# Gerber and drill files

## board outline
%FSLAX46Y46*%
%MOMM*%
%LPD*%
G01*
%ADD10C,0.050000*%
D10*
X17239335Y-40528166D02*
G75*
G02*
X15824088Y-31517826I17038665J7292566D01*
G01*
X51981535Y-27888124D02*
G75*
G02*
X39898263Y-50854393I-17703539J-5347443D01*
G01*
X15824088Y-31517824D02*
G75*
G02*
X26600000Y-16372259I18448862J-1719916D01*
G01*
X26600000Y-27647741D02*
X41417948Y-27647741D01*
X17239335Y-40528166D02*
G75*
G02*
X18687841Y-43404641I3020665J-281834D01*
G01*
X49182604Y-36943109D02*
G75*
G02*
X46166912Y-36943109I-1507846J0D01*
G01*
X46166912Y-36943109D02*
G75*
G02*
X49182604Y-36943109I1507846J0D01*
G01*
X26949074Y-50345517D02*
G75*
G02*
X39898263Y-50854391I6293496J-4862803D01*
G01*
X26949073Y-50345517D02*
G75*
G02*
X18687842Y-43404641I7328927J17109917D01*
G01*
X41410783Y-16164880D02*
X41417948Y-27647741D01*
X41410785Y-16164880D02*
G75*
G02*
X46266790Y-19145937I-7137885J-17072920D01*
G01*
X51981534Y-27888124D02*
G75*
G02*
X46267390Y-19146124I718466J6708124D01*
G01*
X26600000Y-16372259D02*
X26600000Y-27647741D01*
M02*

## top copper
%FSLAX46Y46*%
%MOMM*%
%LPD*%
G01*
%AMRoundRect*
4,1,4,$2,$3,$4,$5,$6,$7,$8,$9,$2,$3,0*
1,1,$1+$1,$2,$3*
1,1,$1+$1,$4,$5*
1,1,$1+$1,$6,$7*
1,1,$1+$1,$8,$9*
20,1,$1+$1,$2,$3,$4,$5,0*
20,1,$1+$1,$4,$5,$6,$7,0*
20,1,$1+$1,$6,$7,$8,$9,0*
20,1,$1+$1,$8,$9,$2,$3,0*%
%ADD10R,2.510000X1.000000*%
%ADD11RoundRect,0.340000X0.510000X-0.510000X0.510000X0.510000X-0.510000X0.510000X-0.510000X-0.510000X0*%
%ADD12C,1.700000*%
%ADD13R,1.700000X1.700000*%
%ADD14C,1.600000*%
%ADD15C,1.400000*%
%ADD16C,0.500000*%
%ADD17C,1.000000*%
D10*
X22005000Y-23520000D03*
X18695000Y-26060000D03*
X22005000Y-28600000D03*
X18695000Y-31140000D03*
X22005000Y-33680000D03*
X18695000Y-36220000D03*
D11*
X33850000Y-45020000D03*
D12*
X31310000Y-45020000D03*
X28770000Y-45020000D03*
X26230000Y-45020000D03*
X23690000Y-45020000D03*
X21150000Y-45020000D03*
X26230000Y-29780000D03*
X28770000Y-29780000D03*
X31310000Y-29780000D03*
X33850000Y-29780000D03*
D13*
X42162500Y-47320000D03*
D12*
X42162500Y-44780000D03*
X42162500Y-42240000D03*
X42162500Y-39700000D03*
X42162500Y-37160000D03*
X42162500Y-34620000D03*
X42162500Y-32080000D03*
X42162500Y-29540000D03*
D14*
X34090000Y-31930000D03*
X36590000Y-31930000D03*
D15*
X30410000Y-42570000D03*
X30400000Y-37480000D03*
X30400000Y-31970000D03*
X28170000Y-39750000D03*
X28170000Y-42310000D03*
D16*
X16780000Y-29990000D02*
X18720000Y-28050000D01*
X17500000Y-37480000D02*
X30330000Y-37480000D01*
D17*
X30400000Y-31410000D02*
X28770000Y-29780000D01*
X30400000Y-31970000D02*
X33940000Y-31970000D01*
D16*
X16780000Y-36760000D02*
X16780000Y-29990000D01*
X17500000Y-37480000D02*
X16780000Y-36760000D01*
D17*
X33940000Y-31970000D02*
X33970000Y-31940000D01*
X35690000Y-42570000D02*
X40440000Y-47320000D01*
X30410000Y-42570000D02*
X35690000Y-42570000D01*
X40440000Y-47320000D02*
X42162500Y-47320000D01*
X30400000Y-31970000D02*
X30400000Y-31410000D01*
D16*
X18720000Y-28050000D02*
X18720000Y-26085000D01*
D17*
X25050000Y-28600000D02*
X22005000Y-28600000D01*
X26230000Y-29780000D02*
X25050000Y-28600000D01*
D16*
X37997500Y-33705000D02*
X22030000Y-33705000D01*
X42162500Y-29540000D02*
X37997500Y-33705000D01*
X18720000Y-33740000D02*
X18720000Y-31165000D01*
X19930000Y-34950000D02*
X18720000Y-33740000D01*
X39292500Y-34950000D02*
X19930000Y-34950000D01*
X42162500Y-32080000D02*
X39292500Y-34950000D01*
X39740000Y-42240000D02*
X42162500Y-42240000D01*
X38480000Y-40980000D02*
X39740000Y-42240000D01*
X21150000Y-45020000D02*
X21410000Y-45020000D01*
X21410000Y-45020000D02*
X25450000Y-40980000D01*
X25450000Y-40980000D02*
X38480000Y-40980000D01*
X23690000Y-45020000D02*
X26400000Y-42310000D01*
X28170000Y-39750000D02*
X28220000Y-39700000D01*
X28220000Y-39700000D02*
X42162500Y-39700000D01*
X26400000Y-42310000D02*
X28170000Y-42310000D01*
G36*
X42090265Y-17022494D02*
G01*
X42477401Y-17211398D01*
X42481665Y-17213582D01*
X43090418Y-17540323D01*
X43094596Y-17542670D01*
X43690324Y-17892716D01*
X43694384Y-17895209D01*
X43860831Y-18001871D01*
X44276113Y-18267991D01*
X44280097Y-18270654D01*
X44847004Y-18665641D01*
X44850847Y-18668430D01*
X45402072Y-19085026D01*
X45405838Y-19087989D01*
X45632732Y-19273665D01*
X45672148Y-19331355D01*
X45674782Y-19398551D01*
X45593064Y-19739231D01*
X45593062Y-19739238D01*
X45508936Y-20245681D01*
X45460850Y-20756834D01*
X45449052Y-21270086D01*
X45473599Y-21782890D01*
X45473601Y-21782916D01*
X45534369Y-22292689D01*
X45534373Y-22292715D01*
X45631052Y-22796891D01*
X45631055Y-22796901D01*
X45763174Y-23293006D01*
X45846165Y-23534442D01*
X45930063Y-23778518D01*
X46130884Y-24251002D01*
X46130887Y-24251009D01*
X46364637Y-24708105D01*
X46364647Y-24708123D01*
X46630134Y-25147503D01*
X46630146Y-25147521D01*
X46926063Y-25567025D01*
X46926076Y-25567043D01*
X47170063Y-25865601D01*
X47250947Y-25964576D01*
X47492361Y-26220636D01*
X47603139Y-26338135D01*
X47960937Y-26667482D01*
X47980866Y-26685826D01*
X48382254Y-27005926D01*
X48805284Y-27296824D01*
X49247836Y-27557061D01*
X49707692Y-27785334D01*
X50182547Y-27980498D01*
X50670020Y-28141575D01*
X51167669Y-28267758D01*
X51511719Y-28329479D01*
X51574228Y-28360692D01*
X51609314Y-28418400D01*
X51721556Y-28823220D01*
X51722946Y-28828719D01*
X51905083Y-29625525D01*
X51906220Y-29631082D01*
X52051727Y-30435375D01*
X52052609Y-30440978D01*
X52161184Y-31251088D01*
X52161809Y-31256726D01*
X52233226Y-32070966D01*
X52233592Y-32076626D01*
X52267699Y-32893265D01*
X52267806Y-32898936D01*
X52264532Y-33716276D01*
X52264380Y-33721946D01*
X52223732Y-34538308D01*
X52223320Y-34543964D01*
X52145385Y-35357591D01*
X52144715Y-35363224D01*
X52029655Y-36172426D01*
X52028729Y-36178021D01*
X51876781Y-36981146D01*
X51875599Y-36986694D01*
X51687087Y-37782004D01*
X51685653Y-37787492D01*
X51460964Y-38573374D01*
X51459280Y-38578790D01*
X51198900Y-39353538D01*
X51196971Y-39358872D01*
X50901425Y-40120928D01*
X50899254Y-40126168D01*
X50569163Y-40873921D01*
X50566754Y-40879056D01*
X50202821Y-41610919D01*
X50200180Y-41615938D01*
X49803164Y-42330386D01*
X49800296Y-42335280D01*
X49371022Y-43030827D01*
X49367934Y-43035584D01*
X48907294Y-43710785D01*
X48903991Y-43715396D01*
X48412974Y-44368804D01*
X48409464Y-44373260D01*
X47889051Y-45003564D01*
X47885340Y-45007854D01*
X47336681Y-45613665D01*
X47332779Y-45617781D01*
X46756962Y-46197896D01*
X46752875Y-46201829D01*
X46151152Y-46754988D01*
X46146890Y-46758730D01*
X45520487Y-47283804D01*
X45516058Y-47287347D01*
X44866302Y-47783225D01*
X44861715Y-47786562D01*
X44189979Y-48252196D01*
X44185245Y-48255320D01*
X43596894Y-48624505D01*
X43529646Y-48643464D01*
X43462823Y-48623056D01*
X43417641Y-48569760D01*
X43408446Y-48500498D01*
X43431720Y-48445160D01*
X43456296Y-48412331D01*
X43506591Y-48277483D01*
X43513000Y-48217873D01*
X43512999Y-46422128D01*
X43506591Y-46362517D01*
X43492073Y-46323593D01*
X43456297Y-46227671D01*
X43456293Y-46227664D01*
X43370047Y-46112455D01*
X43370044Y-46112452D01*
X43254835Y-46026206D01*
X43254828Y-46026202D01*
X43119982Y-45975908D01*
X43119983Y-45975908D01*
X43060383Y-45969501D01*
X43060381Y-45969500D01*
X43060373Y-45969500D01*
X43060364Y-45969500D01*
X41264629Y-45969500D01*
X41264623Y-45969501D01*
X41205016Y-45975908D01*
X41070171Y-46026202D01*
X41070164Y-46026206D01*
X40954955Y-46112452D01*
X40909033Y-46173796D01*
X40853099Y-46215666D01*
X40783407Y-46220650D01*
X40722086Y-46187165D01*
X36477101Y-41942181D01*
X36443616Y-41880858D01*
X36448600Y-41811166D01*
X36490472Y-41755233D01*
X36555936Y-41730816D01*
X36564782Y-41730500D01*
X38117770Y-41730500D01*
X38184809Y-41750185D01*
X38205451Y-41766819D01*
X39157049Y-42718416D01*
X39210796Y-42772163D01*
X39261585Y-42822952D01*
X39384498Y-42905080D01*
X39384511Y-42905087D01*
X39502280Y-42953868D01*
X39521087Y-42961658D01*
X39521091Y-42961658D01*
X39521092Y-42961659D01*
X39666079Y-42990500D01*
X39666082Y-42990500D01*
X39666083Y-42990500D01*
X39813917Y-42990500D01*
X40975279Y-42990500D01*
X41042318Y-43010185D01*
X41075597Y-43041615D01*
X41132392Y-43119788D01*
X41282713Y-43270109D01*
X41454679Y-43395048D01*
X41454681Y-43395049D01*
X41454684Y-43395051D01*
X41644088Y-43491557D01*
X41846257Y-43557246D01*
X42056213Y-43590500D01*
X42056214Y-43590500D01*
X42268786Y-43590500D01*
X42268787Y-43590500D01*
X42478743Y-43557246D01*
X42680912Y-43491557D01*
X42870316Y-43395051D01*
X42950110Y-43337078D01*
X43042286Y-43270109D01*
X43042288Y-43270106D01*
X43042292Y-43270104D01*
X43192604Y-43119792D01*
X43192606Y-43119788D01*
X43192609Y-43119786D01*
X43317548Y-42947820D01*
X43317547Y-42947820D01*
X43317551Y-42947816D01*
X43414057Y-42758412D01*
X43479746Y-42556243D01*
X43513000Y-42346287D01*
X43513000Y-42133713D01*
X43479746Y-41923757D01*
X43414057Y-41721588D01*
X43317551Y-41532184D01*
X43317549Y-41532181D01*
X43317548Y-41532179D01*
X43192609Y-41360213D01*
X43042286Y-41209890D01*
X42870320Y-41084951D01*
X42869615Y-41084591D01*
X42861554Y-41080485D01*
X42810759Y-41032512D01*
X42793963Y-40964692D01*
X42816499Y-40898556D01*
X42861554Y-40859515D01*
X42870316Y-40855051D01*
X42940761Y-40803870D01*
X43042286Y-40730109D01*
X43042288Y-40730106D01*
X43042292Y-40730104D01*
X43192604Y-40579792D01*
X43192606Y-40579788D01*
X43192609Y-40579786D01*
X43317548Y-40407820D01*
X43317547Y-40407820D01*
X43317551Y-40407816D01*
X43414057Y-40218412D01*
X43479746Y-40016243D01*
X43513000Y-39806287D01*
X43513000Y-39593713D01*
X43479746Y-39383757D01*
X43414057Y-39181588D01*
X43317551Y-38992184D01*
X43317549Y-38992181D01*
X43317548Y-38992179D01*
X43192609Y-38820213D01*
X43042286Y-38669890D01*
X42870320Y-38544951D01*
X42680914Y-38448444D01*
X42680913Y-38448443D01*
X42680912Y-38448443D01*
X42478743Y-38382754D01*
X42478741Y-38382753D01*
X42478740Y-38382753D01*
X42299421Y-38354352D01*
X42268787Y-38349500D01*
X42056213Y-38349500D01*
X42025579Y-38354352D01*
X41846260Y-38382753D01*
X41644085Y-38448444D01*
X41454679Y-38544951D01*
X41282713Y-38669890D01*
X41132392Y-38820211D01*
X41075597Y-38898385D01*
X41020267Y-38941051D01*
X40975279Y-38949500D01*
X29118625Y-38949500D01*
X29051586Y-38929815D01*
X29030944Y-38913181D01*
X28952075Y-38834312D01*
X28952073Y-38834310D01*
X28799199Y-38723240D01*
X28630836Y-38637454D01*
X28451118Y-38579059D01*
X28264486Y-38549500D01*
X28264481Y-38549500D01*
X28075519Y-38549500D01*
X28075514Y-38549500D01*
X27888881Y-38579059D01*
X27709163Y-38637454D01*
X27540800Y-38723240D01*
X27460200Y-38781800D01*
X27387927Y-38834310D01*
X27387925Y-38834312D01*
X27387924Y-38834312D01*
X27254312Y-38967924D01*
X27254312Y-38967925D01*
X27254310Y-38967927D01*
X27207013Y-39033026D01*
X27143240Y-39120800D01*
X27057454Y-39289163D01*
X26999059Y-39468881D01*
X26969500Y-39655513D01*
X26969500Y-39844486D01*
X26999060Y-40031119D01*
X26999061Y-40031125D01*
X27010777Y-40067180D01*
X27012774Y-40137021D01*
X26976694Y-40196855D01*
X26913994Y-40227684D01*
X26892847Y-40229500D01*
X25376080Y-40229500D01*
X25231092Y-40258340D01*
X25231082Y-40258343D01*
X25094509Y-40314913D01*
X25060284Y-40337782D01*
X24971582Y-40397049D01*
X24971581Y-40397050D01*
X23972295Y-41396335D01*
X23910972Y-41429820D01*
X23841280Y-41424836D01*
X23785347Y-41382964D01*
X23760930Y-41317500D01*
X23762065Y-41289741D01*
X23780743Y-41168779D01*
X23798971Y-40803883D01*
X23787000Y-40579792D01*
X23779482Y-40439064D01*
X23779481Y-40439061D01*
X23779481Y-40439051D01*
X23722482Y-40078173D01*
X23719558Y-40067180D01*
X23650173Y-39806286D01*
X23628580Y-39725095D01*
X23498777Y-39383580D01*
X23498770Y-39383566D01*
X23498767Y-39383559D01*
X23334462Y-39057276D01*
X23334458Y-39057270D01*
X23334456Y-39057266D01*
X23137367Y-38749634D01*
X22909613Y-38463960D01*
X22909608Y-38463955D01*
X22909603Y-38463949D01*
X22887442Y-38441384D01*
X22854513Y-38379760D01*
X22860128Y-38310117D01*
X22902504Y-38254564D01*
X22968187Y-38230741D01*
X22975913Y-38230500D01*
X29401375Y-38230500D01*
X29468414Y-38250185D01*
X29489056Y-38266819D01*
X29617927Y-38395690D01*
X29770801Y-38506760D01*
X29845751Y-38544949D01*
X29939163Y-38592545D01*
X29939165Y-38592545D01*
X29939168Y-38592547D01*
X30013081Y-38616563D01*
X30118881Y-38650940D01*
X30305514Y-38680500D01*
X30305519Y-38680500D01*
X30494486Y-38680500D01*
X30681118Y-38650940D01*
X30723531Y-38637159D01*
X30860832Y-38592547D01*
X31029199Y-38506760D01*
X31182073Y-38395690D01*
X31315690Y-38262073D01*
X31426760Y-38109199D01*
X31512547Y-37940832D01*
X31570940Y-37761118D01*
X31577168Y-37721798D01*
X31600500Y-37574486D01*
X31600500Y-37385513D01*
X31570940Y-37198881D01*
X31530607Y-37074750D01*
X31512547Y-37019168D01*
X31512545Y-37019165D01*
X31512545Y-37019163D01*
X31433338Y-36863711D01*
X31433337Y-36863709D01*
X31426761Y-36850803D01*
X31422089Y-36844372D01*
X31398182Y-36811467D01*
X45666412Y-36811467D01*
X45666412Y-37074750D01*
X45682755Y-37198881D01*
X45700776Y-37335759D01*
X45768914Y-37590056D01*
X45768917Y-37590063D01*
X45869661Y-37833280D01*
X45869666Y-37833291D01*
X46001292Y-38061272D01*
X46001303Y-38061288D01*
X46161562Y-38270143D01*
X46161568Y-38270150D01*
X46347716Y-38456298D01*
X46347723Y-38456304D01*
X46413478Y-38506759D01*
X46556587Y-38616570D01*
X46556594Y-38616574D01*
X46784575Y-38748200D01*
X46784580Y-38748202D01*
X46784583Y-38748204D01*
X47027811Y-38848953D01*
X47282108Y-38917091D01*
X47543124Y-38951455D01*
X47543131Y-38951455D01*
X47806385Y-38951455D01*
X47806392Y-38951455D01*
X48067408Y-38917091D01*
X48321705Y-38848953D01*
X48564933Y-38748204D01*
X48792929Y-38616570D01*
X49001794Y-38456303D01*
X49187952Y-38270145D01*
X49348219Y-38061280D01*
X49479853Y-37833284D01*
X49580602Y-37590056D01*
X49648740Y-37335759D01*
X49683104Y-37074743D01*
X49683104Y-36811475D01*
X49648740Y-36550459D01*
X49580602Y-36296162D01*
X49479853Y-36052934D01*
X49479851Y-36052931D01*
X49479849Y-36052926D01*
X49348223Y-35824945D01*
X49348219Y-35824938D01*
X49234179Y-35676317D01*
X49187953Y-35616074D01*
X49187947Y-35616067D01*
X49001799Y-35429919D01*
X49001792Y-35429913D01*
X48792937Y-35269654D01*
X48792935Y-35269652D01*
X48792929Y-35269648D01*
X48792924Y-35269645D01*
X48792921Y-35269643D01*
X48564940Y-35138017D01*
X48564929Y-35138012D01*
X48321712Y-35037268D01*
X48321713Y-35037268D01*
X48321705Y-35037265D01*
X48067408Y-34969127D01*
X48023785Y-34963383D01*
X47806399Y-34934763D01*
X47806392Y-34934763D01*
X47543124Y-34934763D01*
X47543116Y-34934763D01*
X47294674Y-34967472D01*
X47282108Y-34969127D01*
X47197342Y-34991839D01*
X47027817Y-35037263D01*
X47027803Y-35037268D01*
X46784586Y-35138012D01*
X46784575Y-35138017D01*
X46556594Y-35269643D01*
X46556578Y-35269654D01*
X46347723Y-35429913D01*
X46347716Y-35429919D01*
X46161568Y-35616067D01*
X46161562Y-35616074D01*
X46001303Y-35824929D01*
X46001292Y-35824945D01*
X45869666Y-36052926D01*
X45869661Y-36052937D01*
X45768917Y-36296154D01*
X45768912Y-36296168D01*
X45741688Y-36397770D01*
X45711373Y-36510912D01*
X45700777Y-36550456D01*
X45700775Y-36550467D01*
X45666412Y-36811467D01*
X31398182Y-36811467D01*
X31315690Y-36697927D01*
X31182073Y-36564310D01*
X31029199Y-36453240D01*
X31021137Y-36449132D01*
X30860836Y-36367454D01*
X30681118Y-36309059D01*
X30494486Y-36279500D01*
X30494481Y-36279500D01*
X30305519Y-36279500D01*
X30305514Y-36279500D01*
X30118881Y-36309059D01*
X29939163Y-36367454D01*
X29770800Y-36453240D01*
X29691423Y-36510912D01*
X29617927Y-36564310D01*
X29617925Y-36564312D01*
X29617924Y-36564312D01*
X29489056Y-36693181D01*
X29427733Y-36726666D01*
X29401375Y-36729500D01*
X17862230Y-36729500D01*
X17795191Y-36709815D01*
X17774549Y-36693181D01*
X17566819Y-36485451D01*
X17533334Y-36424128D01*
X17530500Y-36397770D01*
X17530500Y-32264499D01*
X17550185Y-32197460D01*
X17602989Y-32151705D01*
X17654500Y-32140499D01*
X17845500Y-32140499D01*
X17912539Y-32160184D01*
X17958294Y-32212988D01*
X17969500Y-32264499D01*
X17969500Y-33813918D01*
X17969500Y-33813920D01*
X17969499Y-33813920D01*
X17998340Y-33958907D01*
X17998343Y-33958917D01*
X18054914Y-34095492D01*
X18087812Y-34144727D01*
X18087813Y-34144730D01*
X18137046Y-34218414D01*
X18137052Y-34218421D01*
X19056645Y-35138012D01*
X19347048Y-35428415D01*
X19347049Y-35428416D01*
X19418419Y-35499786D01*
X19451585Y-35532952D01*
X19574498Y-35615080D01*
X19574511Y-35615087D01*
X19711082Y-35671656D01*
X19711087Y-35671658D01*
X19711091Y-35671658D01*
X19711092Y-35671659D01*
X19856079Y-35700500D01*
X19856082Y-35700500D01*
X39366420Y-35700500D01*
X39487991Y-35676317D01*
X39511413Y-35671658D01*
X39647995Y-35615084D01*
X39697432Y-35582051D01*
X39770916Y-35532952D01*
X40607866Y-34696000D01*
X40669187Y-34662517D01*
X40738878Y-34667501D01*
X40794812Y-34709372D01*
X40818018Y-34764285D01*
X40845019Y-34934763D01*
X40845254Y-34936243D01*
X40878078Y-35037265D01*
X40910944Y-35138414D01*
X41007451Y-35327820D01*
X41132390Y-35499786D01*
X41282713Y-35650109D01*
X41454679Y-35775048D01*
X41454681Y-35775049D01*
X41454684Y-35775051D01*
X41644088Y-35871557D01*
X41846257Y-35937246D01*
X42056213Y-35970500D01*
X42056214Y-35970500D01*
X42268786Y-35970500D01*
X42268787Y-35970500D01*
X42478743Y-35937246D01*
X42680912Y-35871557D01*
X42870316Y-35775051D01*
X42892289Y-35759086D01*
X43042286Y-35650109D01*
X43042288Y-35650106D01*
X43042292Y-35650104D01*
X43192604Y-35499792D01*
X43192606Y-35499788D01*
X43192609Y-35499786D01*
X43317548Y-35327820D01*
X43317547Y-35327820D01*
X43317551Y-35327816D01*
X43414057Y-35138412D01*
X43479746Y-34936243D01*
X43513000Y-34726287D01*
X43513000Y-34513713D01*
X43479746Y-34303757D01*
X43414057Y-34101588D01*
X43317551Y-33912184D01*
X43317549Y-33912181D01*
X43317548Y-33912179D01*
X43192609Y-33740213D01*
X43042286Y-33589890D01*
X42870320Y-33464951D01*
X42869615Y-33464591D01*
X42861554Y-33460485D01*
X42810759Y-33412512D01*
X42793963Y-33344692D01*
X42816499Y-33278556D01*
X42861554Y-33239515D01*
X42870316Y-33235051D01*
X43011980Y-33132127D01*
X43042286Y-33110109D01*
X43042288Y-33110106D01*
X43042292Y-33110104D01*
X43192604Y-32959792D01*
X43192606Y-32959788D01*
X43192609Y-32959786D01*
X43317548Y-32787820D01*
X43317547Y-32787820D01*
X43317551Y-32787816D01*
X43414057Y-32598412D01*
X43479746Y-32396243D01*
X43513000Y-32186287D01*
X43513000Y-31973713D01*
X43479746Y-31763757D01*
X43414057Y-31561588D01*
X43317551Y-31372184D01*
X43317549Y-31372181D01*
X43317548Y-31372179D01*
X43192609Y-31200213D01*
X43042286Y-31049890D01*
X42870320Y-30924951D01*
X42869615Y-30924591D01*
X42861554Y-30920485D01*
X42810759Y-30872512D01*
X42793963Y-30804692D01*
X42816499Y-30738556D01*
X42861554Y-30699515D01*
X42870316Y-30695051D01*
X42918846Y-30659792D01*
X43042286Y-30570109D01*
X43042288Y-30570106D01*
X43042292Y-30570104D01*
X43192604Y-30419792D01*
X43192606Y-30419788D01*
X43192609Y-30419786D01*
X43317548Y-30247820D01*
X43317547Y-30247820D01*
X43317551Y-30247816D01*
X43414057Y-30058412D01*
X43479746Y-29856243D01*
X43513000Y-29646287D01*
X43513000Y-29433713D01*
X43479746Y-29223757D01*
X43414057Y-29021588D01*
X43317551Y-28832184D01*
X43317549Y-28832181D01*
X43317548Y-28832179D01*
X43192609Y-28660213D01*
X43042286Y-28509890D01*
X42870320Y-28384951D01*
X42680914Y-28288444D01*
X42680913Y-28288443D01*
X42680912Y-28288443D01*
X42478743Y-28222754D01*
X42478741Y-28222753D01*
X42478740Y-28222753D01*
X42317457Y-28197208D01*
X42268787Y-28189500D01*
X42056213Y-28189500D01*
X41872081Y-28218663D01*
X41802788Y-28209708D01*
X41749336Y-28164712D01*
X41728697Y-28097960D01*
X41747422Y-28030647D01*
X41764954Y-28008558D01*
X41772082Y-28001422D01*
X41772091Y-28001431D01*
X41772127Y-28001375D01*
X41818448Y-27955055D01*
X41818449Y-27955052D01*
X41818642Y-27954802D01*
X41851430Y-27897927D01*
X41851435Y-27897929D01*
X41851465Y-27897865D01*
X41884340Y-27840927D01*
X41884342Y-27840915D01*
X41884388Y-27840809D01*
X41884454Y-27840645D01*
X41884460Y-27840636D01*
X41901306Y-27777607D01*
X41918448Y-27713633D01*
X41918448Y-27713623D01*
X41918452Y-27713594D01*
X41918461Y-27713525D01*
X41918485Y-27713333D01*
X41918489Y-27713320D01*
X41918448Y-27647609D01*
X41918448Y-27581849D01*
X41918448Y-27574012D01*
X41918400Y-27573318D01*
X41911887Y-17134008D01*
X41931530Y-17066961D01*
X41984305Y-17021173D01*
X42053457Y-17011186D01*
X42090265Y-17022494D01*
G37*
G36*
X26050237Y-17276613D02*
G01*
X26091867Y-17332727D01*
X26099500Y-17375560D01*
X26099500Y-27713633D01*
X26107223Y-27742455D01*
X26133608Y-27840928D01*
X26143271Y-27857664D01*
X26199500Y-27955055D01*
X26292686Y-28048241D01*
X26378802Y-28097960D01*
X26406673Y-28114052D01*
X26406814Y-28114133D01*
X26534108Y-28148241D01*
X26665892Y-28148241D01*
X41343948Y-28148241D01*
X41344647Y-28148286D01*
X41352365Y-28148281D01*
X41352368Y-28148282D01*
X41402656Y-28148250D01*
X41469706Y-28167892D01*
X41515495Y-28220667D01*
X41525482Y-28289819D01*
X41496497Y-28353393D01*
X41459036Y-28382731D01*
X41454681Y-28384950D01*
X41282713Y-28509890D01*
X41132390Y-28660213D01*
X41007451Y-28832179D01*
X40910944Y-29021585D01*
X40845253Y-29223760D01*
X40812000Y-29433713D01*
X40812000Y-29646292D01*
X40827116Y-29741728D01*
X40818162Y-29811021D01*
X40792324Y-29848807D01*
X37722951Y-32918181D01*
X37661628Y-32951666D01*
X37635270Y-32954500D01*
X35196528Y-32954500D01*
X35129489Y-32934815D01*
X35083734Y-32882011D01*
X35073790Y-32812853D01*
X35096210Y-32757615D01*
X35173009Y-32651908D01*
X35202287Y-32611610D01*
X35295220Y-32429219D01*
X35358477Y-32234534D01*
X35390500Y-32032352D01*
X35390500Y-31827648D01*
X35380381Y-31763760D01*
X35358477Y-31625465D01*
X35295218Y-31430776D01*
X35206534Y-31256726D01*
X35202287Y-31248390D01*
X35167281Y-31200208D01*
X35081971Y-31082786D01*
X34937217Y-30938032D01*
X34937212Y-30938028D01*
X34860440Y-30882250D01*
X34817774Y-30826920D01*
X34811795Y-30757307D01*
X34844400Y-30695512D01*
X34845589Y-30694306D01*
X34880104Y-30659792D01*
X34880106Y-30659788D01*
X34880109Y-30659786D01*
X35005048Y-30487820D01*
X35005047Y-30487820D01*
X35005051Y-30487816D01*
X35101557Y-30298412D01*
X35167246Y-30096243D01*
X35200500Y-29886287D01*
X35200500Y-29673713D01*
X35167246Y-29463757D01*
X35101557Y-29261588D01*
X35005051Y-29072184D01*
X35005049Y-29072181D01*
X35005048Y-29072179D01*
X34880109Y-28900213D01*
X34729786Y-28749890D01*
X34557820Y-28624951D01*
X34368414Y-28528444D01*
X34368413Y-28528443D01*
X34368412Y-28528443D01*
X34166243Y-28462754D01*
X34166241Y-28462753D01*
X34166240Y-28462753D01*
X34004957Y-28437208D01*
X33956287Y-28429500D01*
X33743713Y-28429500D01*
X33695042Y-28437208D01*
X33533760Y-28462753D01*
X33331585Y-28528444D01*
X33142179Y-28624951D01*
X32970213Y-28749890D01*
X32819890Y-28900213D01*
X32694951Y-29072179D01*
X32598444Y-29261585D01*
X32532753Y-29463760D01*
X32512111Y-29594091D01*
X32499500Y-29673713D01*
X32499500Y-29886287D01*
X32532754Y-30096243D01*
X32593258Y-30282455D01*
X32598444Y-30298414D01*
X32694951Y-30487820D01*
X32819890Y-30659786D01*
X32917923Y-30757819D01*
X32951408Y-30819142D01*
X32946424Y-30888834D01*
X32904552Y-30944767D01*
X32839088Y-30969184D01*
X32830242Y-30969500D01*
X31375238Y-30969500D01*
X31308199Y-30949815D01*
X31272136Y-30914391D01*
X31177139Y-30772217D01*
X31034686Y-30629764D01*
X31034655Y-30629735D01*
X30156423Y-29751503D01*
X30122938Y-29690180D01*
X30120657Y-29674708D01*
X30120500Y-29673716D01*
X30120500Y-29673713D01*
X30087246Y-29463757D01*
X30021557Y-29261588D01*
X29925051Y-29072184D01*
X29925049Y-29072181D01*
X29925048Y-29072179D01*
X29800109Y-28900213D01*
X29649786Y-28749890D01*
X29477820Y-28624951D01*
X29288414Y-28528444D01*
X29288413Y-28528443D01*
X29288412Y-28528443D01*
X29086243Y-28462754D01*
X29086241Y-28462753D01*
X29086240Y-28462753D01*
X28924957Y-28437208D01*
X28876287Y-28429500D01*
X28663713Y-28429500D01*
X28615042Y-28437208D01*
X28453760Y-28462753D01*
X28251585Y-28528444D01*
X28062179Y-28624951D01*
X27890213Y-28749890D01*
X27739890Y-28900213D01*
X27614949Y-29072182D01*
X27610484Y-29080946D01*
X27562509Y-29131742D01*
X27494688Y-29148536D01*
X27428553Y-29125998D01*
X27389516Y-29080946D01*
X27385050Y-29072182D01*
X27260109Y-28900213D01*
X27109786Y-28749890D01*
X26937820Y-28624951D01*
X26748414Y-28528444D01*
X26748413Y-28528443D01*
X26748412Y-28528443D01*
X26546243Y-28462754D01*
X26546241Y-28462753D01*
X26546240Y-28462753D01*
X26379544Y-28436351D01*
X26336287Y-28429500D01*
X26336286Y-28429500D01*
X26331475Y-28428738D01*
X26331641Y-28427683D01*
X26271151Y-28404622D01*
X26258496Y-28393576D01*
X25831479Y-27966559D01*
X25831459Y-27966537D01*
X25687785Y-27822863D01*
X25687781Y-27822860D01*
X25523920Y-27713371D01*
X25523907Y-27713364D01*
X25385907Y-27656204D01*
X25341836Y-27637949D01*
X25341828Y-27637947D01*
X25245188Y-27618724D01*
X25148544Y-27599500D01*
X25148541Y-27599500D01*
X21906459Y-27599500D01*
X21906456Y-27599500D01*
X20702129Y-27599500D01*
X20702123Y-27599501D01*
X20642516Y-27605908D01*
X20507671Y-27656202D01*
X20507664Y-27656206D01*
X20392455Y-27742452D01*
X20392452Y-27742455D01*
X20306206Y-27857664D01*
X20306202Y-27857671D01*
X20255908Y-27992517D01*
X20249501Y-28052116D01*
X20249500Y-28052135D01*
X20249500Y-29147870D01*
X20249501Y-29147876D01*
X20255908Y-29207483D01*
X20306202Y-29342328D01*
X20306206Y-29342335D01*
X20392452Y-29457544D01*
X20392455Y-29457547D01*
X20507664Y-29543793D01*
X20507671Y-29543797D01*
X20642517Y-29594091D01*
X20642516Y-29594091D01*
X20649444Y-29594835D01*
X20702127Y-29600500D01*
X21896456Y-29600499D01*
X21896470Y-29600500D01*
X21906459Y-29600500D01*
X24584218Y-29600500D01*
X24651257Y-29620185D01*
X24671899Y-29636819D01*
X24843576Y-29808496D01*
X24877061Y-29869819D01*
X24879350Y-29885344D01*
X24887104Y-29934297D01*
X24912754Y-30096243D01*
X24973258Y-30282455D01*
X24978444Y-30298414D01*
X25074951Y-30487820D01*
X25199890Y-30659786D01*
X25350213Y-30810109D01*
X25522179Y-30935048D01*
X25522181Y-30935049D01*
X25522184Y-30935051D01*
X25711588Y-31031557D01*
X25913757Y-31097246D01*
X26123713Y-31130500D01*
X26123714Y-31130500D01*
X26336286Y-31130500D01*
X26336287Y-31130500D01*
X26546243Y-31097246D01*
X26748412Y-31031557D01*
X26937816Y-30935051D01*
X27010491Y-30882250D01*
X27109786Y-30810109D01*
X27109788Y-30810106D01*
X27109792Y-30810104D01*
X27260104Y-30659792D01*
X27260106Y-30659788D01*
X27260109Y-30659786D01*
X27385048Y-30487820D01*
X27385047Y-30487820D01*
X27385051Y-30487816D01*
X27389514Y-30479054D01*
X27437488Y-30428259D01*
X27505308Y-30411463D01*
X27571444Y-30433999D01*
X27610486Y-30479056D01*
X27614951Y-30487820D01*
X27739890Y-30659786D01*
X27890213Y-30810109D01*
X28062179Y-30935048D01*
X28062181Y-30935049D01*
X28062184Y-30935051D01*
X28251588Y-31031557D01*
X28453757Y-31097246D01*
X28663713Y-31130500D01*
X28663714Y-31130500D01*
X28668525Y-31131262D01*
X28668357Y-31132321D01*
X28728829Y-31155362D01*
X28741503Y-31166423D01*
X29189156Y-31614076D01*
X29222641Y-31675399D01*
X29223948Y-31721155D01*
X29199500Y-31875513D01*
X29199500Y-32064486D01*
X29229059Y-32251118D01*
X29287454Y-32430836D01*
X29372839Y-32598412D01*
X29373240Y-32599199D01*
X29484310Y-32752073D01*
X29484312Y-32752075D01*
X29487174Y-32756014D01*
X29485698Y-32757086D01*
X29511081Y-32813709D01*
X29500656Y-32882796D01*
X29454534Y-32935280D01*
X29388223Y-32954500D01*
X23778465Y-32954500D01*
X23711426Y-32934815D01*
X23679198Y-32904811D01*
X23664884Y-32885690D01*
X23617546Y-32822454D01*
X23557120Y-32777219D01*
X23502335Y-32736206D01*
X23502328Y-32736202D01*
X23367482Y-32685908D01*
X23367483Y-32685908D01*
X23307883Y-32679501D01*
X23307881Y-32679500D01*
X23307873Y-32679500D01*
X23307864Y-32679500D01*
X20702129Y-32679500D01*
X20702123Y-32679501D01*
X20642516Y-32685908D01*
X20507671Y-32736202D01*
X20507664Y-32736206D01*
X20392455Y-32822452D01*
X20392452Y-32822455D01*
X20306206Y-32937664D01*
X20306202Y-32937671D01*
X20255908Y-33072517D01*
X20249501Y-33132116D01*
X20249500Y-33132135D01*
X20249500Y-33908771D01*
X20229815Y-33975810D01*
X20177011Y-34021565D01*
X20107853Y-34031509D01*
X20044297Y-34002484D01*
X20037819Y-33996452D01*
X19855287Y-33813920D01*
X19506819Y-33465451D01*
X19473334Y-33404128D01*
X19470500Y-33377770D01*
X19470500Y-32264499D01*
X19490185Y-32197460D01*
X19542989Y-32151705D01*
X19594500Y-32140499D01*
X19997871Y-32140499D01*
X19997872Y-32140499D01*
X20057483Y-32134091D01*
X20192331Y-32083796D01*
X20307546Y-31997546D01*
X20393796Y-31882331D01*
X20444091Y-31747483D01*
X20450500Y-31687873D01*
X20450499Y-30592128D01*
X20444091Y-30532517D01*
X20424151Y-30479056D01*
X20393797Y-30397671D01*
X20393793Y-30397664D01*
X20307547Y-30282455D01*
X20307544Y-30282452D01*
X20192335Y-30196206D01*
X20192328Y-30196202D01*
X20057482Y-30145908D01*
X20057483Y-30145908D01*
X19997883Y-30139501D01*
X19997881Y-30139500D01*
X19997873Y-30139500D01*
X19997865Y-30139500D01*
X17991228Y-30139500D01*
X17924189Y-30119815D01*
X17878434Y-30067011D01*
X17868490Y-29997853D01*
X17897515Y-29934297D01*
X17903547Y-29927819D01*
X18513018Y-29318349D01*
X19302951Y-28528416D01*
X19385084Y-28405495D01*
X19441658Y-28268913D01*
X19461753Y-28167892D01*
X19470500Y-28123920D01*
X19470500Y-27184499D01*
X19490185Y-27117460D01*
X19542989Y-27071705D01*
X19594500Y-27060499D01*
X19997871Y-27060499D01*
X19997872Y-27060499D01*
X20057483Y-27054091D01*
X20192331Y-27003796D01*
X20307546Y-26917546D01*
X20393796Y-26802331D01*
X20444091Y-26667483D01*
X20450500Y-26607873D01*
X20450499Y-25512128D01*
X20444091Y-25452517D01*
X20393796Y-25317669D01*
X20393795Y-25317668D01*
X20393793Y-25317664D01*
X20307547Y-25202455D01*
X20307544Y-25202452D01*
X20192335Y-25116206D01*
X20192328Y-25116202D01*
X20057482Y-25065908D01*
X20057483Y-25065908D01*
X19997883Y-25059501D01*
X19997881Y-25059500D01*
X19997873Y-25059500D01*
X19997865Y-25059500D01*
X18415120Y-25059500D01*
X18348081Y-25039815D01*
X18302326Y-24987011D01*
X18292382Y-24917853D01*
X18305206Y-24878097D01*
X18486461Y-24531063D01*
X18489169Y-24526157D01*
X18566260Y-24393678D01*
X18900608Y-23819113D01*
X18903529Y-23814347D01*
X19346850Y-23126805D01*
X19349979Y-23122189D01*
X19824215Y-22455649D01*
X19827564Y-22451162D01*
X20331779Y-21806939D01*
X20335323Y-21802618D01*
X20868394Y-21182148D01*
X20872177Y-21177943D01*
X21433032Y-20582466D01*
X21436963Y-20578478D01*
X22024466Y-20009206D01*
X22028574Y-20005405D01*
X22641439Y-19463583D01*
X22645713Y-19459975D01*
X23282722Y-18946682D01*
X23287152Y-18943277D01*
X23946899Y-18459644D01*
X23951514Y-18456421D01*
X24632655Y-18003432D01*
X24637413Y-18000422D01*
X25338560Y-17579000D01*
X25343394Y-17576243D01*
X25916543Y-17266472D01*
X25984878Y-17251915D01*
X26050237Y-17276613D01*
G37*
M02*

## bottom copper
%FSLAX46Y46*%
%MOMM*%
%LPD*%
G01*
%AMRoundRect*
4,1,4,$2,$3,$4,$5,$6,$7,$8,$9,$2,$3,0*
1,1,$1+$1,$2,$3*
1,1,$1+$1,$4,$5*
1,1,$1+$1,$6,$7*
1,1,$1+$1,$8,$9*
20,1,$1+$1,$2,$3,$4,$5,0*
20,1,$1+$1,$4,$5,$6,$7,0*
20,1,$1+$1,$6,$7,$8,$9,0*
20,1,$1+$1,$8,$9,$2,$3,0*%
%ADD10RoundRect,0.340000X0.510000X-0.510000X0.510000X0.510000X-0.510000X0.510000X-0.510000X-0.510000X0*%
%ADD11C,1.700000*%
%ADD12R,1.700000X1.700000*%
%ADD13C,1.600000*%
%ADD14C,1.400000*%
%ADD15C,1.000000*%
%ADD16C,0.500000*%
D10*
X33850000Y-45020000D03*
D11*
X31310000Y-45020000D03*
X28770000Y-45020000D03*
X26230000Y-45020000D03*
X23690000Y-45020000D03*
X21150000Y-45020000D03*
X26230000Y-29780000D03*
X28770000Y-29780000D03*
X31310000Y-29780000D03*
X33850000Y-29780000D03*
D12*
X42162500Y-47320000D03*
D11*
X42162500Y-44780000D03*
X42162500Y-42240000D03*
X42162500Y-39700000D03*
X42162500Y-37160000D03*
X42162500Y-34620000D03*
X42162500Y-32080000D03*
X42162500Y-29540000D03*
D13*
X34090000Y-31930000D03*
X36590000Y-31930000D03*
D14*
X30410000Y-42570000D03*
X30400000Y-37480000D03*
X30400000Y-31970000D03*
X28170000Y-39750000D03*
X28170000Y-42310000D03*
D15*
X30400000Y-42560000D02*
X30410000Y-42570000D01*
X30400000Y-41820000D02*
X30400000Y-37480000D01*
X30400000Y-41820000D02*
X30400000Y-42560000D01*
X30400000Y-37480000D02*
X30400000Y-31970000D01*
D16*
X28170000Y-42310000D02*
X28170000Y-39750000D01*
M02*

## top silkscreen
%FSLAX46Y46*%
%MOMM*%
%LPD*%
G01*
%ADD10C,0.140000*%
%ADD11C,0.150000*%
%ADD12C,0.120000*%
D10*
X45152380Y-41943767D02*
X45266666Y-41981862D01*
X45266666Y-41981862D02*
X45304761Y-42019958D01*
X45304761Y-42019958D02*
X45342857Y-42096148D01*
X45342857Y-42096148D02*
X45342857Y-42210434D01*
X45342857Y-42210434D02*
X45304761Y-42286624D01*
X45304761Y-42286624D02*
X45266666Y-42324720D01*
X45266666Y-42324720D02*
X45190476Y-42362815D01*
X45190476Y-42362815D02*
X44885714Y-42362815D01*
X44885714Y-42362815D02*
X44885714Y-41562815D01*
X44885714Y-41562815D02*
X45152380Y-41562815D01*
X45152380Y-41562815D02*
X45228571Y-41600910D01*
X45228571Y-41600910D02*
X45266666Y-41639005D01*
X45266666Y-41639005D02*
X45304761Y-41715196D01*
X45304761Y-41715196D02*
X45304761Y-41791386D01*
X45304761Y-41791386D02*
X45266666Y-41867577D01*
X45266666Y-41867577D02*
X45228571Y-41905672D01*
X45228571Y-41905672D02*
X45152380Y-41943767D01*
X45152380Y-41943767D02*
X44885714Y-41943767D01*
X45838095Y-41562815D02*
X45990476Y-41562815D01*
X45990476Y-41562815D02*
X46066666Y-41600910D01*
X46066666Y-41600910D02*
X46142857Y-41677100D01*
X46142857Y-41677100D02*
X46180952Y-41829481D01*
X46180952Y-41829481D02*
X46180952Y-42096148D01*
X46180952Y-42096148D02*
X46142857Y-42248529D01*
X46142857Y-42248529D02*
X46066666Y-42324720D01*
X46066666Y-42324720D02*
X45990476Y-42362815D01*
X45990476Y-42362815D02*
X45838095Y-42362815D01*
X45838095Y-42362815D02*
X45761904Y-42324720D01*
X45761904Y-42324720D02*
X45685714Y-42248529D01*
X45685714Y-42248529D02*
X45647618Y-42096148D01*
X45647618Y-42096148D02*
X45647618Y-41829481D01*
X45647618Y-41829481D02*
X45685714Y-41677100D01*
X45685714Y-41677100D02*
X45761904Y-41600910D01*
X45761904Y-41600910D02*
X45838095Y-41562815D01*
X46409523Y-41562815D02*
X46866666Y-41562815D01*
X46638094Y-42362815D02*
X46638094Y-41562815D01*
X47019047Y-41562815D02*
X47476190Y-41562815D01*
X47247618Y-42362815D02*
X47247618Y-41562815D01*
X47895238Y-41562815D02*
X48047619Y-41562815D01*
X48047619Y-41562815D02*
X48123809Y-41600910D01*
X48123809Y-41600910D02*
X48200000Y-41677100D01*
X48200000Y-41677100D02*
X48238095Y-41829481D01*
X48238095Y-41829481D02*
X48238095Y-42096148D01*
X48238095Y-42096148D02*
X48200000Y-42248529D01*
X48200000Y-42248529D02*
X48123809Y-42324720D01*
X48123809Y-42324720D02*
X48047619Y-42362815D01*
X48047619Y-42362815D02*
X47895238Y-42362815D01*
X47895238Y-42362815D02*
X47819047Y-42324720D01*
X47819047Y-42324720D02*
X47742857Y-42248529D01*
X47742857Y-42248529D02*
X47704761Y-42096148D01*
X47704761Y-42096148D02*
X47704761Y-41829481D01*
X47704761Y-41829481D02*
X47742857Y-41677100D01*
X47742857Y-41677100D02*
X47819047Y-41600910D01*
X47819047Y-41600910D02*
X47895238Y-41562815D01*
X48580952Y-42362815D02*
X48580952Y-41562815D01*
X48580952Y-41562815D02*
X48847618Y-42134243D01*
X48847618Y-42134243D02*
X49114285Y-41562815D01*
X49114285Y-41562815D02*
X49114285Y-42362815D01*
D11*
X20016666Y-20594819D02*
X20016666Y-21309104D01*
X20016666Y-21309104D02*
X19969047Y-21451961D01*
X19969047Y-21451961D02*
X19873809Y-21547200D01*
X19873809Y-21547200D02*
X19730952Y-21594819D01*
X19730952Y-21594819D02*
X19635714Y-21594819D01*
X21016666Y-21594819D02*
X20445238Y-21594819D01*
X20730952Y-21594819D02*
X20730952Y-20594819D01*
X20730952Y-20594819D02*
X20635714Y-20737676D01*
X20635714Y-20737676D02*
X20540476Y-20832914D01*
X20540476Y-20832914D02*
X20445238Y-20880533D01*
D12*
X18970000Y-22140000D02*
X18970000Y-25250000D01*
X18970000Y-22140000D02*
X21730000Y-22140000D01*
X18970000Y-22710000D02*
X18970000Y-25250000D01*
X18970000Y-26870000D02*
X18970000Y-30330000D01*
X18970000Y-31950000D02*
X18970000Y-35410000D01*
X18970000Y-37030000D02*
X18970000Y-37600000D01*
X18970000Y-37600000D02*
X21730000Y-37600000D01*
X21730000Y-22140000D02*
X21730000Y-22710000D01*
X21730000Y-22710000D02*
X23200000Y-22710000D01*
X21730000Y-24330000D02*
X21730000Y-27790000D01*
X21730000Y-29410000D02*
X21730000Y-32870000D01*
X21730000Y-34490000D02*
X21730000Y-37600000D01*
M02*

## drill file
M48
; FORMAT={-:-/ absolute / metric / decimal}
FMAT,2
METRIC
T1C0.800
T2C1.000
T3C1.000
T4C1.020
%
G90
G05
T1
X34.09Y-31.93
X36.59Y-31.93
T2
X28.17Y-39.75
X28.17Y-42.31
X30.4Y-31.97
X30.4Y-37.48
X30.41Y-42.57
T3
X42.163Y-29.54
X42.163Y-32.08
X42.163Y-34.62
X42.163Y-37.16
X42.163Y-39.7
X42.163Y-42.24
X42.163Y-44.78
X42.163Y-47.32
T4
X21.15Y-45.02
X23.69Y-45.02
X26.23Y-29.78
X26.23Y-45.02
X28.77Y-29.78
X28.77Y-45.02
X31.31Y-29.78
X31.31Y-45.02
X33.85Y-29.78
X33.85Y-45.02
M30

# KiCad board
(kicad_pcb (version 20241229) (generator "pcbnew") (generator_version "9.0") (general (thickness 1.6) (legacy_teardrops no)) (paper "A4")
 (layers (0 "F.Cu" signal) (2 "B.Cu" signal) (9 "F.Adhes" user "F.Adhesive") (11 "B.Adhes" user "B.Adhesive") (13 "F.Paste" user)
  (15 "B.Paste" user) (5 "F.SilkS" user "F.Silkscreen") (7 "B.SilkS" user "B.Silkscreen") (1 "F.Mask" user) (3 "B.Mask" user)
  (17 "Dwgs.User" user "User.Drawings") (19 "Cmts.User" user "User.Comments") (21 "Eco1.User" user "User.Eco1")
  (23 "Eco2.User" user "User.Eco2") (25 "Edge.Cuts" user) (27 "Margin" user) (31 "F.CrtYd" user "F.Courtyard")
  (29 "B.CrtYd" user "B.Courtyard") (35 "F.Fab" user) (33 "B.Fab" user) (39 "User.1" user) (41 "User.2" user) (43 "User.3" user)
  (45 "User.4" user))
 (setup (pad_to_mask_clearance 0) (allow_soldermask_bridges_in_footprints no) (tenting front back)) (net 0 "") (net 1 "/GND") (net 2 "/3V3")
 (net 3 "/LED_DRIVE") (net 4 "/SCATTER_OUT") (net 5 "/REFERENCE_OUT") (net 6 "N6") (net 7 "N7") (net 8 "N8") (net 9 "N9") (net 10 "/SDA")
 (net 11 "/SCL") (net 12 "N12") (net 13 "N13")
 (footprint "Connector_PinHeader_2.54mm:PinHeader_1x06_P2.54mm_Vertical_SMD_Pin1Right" (layer "F.Cu") (at 20.35 29.87)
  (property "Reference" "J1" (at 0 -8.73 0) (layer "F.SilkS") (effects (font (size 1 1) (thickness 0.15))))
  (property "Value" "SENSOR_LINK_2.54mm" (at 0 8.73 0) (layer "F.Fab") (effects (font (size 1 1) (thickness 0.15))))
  (fp_line (start -1.38 -7.73) (end -1.38 -4.62) (stroke (width 0.12) (type solid)) (layer "F.SilkS"))
  (fp_line (start -1.38 -7.73) (end 1.38 -7.73) (stroke (width 0.12) (type solid)) (layer "F.SilkS"))
  (fp_line (start -1.38 -7.16) (end -1.38 -4.62) (stroke (width 0.12) (type solid)) (layer "F.SilkS"))
  (fp_line (start -1.38 -3) (end -1.38 0.46) (stroke (width 0.12) (type solid)) (layer "F.SilkS"))
  (fp_line (start -1.38 2.08) (end -1.38 5.54) (stroke (width 0.12) (type solid)) (layer "F.SilkS"))
  (fp_line (start -1.38 7.16) (end -1.38 7.73) (stroke (width 0.12) (type solid)) (layer "F.SilkS"))
  (fp_line (start -1.38 7.73) (end 1.38 7.73) (stroke (width 0.12) (type solid)) (layer "F.SilkS"))
  (fp_line (start 1.38 -7.73) (end 1.38 -7.16) (stroke (width 0.12) (type solid)) (layer "F.SilkS"))
  (fp_line (start 1.38 -7.16) (end 2.85 -7.16) (stroke (width 0.12) (type solid)) (layer "F.SilkS"))
  (fp_line (start 1.38 -5.54) (end 1.38 -2.08) (stroke (width 0.12) (type solid)) (layer "F.SilkS"))
  (fp_line (start 1.38 -0.46) (end 1.38 3) (stroke (width 0.12) (type solid)) (layer "F.SilkS"))
  (fp_line (start 1.38 4.62) (end 1.38 7.73) (stroke (width 0.12) (type solid)) (layer "F.SilkS"))
  (pad "1" smd rect (at 1.655 -6.35) (size 2.51 1) (layers "F.Cu" "F.Mask" "F.Paste") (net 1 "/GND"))
  (pad "2" smd rect (at -1.655 -3.81) (size 2.51 1) (layers "F.Cu" "F.Mask" "F.Paste") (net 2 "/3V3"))
  (pad "3" smd rect (at 1.655 -1.27) (size 2.51 1) (layers "F.Cu" "F.Mask" "F.Paste") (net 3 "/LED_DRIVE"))
  (pad "4" smd rect (at -1.655 1.27) (size 2.51 1) (layers "F.Cu" "F.Mask" "F.Paste") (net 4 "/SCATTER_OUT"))
  (pad "5" smd rect (at 1.655 3.81) (size 2.51 1) (layers "F.Cu" "F.Mask" "F.Paste") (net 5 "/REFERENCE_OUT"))
  (pad "6" smd rect (at -1.655 6.35) (size 2.51 1) (layers "F.Cu" "F.Mask" "F.Paste") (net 1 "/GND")))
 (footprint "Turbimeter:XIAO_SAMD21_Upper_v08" (layer "B.Cu") (at 26.23 37.4 90)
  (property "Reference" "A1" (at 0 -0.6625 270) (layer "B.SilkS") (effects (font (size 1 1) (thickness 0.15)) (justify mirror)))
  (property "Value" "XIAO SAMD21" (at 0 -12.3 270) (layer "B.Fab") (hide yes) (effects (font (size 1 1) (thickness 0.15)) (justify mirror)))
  (pad "1" thru_hole roundrect (at -7.62 7.62 90) (size 1.7 1.7) (drill 1.02) (layers "*.Cu" "*.Mask") (remove_unused_layers no)
   (roundrect_rratio 0.2) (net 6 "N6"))
  (pad "2" thru_hole circle (at -7.62 5.08 90) (size 1.7 1.7) (drill 1.02) (layers "*.Cu" "*.Mask") (remove_unused_layers no) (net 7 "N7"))
  (pad "3" thru_hole circle (at -7.62 2.54 90) (size 1.7 1.7) (drill 1.02) (layers "*.Cu" "*.Mask") (remove_unused_layers no) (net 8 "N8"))
  (pad "4" thru_hole circle (at -7.62 0 90) (size 1.7 1.7) (drill 1.02) (layers "*.Cu" "*.Mask") (remove_unused_layers no) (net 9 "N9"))
  (pad "5" thru_hole circle (at -7.62 -2.54 90) (size 1.7 1.7) (drill 1.02) (layers "*.Cu" "*.Mask") (remove_unused_layers no)
   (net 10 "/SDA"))
  (pad "6" thru_hole circle (at -7.62 -5.08 90) (size 1.7 1.7) (drill 1.02) (layers "*.Cu" "*.Mask") (remove_unused_layers no)
   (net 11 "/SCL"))
  (pad "11" thru_hole circle (at 7.62 0 90) (size 1.7 1.7) (drill 1.02) (layers "*.Cu" "*.Mask") (remove_unused_layers no)
   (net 3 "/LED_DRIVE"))
  (pad "12" thru_hole circle (at 7.62 2.54 90) (size 1.7 1.7) (drill 1.02) (layers "*.Cu" "*.Mask") (remove_unused_layers no) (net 2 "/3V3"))
  (pad "13" thru_hole circle (at 7.62 5.08 90) (size 1.7 1.7) (drill 1.02) (layers "*.Cu" "*.Mask") (remove_unused_layers no) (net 1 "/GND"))
  (pad "14" thru_hole circle (at 7.62 7.62 90) (size 1.7 1.7) (drill 1.02) (layers "*.Cu" "*.Mask") (remove_unused_layers no) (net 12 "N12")))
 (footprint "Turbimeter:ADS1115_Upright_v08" (layer "B.Cu") (at 42.1625 47.32 90)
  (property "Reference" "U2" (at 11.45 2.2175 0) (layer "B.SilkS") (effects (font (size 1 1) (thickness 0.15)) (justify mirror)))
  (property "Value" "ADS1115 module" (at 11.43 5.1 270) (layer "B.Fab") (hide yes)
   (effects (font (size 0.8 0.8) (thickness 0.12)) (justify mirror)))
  (pad "1" thru_hole rect (at 0 0 90) (size 1.7 1.7) (drill 1) (layers "*.Cu" "*.Mask") (remove_unused_layers no) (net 2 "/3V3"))
  (pad "2" thru_hole circle (at 2.54 0 90) (size 1.7 1.7) (drill 1) (layers "*.Cu" "*.Mask") (remove_unused_layers no) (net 1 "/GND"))
  (pad "3" thru_hole circle (at 5.08 0 90) (size 1.7 1.7) (drill 1) (layers "*.Cu" "*.Mask") (remove_unused_layers no) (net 11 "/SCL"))
  (pad "4" thru_hole circle (at 7.62 0 90) (size 1.7 1.7) (drill 1) (layers "*.Cu" "*.Mask") (remove_unused_layers no) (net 10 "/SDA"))
  (pad "5" thru_hole circle (at 10.16 0 90) (size 1.7 1.7) (drill 1) (layers "*.Cu" "*.Mask") (remove_unused_layers no) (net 1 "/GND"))
  (pad "6" thru_hole circle (at 12.7 0 90) (size 1.7 1.7) (drill 1) (layers "*.Cu" "*.Mask") (remove_unused_layers no) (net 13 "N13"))
  (pad "7" thru_hole circle (at 15.24 0 90) (size 1.7 1.7) (drill 1) (layers "*.Cu" "*.Mask") (remove_unused_layers no)
   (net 4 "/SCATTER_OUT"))
  (pad "8" thru_hole circle (at 17.78 0 90) (size 1.7 1.7) (drill 1) (layers "*.Cu" "*.Mask") (remove_unused_layers no)
   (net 5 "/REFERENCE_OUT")))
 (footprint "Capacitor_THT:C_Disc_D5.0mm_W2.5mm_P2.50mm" (layer "B.Cu") (at 34.09 31.93)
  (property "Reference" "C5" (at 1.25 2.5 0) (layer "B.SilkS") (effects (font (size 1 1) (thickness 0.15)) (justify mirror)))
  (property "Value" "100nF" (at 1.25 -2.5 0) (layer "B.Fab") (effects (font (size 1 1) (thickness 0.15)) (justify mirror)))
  (pad "1" thru_hole circle (at 0 0) (size 1.6 1.6) (drill 0.8) (layers "*.Cu" "*.Mask") (remove_unused_layers no) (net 2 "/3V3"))
  (pad "2" thru_hole circle (at 2.5 0) (size 1.6 1.6) (drill 0.8) (layers "*.Cu" "*.Mask") (remove_unused_layers no) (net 1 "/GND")))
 (gr_arc (start 17.239335 40.528166) (mid 15.968786 36.111414) (end 15.824088 31.517826) (stroke (width 0.05) (type default))
  (layer "Edge.Cuts"))
 (gr_arc (start 51.981535 27.888124) (mid 50.644497 41.846495) (end 39.898263 50.854393) (stroke (width 0.05) (type default))
  (layer "Edge.Cuts"))
 (gr_arc (start 15.824088 31.517824) (mid 19.175457 22.496031) (end 26.6 16.372259) (stroke (width 0.05) (type default)) (layer "Edge.Cuts"))
 (gr_line (start 26.6 27.647741) (end 41.417948 27.647741) (stroke (width 0.05) (type default)) (layer "Edge.Cuts"))
 (gr_arc (start 17.239335 40.528166) (mid 22.969619 39.445518) (end 18.687841 43.404641) (stroke (width 0.05) (type default))
  (layer "Edge.Cuts"))
 (gr_circle (center 47.674758 36.943109) (end 49.074758 37.503109) (stroke (width 0.05) (type default)) (fill no) (layer "Edge.Cuts"))
 (gr_arc (start 26.949074 50.345517) (mid 33.554876 47.261156) (end 39.898263 50.854391) (stroke (width 0.05) (type default))
  (layer "Edge.Cuts"))
 (gr_arc (start 26.949073 50.345517) (mid 22.304485 47.486824) (end 18.687842 43.404641) (stroke (width 0.05) (type default))
  (layer "Edge.Cuts"))
 (gr_line (start 41.410783 16.16488) (end 41.417948 27.647741) (stroke (width 0.05) (type default)) (layer "Edge.Cuts"))
 (gr_arc (start 41.410785 16.16488) (mid 43.954217 17.467379) (end 46.266792 19.145935) (stroke (width 0.05) (type default))
  (layer "Edge.Cuts"))
 (gr_arc (start 51.981534 27.888124) (mid 47.052867 24.871207) (end 46.26739 19.146124) (stroke (width 0.05) (type default))
  (layer "Edge.Cuts"))
 (gr_line (start 26.6 16.372259) (end 26.6 27.647741) (stroke (width 0.05) (type default)) (layer "Edge.Cuts"))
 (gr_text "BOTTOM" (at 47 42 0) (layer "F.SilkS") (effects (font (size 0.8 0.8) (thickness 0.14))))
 (segment (start 16.78 29.99) (end 18.72 28.05) (width 0.5) (layer "F.Cu") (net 2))
 (segment (start 17.5 37.48) (end 30.33 37.48) (width 0.5) (layer "F.Cu") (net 2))
 (segment (start 30.4 31.41) (end 28.77 29.78) (width 1) (layer "F.Cu") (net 2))
 (segment (start 30.4 31.97) (end 33.94 31.97) (width 1) (layer "F.Cu") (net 2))
 (segment (start 16.78 36.76) (end 16.78 29.99) (width 0.5) (layer "F.Cu") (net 2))
 (segment (start 17.5 37.48) (end 16.78 36.76) (width 0.5) (layer "F.Cu") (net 2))
 (segment (start 33.94 31.97) (end 33.97 31.94) (width 1) (layer "F.Cu") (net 2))
 (segment (start 35.69 42.57) (end 40.44 47.32) (width 1) (layer "F.Cu") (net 2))
 (segment (start 30.41 42.57) (end 35.69 42.57) (width 1) (layer "F.Cu") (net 2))
 (segment (start 40.44 47.32) (end 42.1625 47.32) (width 1) (layer "F.Cu") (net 2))
 (segment (start 30.4 31.97) (end 30.4 31.41) (width 1) (layer "F.Cu") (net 2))
 (segment (start 18.72 28.05) (end 18.72 26.085) (width 0.5) (layer "F.Cu") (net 2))
 (via (at 30.41 42.57) (size 1.4) (drill 1) (layers "F.Cu" "B.Cu") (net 2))
 (via (at 30.4 37.48) (size 1.4) (drill 1) (layers "F.Cu" "B.Cu") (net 2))
 (via (at 30.4 31.97) (size 1.4) (drill 1) (layers "F.Cu" "B.Cu") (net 2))
 (segment (start 30.4 42.56) (end 30.41 42.57) (width 1) (layer "B.Cu") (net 2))
 (segment (start 30.4 41.82) (end 30.4 37.48) (width 1) (layer "B.Cu") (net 2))
 (segment (start 30.4 41.82) (end 30.4 42.56) (width 1) (layer "B.Cu") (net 2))
 (segment (start 30.4 37.48) (end 30.4 31.97) (width 1) (layer "B.Cu") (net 2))
 (segment (start 25.05 28.6) (end 22.005 28.6) (width 1) (layer "F.Cu") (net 3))
 (segment (start 26.23 29.78) (end 25.05 28.6) (width 1) (layer "F.Cu") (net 3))
 (segment (start 37.9975 33.705) (end 22.03 33.705) (width 0.5) (layer "F.Cu") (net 5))
 (segment (start 42.1625 29.54) (end 37.9975 33.705) (width 0.5) (layer "F.Cu") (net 5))
 (segment (start 18.72 33.74) (end 18.72 31.165) (width 0.5) (layer "F.Cu") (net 4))
 (segment (start 19.93 34.95) (end 18.72 33.74) (width 0.5) (layer "F.Cu") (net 4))
 (segment (start 39.2925 34.95) (end 19.93 34.95) (width 0.5) (layer "F.Cu") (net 4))
 (segment (start 42.1625 32.08) (end 39.2925 34.95) (width 0.5) (layer "F.Cu") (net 4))
 (segment (start 39.74 42.24) (end 42.1625 42.24) (width 0.5) (layer "F.Cu") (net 11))
 (segment (start 38.48 40.98) (end 39.74 42.24) (width 0.5) (layer "F.Cu") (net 11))
 (segment (start 21.15 45.02) (end 21.41 45.02) (width 0.5) (layer "F.Cu") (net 11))
 (segment (start 21.41 45.02) (end 25.45 40.98) (width 0.5) (layer "F.Cu") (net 11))
 (segment (start 25.45 40.98) (end 38.48 40.98) (width 0.5) (layer "F.Cu") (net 11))
 (segment (start 23.69 45.02) (end 26.4 42.31) (width 0.5) (layer "F.Cu") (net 10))
 (segment (start 28.17 39.75) (end 28.22 39.7) (width 0.5) (layer "F.Cu") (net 10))
 (segment (start 28.22 39.7) (end 42.1625 39.7) (width 0.5) (layer "F.Cu") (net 10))
 (segment (start 26.4 42.31) (end 28.17 42.31) (width 0.5) (layer "F.Cu") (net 10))
 (via (at 28.17 39.75) (size 1.4) (drill 1) (layers "F.Cu" "B.Cu") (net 10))
 (via (at 28.17 42.31) (size 1.4) (drill 1) (layers "F.Cu" "B.Cu") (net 10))
 (segment (start 28.17 42.31) (end 28.17 39.75) (width 0.5) (layer "B.Cu") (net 10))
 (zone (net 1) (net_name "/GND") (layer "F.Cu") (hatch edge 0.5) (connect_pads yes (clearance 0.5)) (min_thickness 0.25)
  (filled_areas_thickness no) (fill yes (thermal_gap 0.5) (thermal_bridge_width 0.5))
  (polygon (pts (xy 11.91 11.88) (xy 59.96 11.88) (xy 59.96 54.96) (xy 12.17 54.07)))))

